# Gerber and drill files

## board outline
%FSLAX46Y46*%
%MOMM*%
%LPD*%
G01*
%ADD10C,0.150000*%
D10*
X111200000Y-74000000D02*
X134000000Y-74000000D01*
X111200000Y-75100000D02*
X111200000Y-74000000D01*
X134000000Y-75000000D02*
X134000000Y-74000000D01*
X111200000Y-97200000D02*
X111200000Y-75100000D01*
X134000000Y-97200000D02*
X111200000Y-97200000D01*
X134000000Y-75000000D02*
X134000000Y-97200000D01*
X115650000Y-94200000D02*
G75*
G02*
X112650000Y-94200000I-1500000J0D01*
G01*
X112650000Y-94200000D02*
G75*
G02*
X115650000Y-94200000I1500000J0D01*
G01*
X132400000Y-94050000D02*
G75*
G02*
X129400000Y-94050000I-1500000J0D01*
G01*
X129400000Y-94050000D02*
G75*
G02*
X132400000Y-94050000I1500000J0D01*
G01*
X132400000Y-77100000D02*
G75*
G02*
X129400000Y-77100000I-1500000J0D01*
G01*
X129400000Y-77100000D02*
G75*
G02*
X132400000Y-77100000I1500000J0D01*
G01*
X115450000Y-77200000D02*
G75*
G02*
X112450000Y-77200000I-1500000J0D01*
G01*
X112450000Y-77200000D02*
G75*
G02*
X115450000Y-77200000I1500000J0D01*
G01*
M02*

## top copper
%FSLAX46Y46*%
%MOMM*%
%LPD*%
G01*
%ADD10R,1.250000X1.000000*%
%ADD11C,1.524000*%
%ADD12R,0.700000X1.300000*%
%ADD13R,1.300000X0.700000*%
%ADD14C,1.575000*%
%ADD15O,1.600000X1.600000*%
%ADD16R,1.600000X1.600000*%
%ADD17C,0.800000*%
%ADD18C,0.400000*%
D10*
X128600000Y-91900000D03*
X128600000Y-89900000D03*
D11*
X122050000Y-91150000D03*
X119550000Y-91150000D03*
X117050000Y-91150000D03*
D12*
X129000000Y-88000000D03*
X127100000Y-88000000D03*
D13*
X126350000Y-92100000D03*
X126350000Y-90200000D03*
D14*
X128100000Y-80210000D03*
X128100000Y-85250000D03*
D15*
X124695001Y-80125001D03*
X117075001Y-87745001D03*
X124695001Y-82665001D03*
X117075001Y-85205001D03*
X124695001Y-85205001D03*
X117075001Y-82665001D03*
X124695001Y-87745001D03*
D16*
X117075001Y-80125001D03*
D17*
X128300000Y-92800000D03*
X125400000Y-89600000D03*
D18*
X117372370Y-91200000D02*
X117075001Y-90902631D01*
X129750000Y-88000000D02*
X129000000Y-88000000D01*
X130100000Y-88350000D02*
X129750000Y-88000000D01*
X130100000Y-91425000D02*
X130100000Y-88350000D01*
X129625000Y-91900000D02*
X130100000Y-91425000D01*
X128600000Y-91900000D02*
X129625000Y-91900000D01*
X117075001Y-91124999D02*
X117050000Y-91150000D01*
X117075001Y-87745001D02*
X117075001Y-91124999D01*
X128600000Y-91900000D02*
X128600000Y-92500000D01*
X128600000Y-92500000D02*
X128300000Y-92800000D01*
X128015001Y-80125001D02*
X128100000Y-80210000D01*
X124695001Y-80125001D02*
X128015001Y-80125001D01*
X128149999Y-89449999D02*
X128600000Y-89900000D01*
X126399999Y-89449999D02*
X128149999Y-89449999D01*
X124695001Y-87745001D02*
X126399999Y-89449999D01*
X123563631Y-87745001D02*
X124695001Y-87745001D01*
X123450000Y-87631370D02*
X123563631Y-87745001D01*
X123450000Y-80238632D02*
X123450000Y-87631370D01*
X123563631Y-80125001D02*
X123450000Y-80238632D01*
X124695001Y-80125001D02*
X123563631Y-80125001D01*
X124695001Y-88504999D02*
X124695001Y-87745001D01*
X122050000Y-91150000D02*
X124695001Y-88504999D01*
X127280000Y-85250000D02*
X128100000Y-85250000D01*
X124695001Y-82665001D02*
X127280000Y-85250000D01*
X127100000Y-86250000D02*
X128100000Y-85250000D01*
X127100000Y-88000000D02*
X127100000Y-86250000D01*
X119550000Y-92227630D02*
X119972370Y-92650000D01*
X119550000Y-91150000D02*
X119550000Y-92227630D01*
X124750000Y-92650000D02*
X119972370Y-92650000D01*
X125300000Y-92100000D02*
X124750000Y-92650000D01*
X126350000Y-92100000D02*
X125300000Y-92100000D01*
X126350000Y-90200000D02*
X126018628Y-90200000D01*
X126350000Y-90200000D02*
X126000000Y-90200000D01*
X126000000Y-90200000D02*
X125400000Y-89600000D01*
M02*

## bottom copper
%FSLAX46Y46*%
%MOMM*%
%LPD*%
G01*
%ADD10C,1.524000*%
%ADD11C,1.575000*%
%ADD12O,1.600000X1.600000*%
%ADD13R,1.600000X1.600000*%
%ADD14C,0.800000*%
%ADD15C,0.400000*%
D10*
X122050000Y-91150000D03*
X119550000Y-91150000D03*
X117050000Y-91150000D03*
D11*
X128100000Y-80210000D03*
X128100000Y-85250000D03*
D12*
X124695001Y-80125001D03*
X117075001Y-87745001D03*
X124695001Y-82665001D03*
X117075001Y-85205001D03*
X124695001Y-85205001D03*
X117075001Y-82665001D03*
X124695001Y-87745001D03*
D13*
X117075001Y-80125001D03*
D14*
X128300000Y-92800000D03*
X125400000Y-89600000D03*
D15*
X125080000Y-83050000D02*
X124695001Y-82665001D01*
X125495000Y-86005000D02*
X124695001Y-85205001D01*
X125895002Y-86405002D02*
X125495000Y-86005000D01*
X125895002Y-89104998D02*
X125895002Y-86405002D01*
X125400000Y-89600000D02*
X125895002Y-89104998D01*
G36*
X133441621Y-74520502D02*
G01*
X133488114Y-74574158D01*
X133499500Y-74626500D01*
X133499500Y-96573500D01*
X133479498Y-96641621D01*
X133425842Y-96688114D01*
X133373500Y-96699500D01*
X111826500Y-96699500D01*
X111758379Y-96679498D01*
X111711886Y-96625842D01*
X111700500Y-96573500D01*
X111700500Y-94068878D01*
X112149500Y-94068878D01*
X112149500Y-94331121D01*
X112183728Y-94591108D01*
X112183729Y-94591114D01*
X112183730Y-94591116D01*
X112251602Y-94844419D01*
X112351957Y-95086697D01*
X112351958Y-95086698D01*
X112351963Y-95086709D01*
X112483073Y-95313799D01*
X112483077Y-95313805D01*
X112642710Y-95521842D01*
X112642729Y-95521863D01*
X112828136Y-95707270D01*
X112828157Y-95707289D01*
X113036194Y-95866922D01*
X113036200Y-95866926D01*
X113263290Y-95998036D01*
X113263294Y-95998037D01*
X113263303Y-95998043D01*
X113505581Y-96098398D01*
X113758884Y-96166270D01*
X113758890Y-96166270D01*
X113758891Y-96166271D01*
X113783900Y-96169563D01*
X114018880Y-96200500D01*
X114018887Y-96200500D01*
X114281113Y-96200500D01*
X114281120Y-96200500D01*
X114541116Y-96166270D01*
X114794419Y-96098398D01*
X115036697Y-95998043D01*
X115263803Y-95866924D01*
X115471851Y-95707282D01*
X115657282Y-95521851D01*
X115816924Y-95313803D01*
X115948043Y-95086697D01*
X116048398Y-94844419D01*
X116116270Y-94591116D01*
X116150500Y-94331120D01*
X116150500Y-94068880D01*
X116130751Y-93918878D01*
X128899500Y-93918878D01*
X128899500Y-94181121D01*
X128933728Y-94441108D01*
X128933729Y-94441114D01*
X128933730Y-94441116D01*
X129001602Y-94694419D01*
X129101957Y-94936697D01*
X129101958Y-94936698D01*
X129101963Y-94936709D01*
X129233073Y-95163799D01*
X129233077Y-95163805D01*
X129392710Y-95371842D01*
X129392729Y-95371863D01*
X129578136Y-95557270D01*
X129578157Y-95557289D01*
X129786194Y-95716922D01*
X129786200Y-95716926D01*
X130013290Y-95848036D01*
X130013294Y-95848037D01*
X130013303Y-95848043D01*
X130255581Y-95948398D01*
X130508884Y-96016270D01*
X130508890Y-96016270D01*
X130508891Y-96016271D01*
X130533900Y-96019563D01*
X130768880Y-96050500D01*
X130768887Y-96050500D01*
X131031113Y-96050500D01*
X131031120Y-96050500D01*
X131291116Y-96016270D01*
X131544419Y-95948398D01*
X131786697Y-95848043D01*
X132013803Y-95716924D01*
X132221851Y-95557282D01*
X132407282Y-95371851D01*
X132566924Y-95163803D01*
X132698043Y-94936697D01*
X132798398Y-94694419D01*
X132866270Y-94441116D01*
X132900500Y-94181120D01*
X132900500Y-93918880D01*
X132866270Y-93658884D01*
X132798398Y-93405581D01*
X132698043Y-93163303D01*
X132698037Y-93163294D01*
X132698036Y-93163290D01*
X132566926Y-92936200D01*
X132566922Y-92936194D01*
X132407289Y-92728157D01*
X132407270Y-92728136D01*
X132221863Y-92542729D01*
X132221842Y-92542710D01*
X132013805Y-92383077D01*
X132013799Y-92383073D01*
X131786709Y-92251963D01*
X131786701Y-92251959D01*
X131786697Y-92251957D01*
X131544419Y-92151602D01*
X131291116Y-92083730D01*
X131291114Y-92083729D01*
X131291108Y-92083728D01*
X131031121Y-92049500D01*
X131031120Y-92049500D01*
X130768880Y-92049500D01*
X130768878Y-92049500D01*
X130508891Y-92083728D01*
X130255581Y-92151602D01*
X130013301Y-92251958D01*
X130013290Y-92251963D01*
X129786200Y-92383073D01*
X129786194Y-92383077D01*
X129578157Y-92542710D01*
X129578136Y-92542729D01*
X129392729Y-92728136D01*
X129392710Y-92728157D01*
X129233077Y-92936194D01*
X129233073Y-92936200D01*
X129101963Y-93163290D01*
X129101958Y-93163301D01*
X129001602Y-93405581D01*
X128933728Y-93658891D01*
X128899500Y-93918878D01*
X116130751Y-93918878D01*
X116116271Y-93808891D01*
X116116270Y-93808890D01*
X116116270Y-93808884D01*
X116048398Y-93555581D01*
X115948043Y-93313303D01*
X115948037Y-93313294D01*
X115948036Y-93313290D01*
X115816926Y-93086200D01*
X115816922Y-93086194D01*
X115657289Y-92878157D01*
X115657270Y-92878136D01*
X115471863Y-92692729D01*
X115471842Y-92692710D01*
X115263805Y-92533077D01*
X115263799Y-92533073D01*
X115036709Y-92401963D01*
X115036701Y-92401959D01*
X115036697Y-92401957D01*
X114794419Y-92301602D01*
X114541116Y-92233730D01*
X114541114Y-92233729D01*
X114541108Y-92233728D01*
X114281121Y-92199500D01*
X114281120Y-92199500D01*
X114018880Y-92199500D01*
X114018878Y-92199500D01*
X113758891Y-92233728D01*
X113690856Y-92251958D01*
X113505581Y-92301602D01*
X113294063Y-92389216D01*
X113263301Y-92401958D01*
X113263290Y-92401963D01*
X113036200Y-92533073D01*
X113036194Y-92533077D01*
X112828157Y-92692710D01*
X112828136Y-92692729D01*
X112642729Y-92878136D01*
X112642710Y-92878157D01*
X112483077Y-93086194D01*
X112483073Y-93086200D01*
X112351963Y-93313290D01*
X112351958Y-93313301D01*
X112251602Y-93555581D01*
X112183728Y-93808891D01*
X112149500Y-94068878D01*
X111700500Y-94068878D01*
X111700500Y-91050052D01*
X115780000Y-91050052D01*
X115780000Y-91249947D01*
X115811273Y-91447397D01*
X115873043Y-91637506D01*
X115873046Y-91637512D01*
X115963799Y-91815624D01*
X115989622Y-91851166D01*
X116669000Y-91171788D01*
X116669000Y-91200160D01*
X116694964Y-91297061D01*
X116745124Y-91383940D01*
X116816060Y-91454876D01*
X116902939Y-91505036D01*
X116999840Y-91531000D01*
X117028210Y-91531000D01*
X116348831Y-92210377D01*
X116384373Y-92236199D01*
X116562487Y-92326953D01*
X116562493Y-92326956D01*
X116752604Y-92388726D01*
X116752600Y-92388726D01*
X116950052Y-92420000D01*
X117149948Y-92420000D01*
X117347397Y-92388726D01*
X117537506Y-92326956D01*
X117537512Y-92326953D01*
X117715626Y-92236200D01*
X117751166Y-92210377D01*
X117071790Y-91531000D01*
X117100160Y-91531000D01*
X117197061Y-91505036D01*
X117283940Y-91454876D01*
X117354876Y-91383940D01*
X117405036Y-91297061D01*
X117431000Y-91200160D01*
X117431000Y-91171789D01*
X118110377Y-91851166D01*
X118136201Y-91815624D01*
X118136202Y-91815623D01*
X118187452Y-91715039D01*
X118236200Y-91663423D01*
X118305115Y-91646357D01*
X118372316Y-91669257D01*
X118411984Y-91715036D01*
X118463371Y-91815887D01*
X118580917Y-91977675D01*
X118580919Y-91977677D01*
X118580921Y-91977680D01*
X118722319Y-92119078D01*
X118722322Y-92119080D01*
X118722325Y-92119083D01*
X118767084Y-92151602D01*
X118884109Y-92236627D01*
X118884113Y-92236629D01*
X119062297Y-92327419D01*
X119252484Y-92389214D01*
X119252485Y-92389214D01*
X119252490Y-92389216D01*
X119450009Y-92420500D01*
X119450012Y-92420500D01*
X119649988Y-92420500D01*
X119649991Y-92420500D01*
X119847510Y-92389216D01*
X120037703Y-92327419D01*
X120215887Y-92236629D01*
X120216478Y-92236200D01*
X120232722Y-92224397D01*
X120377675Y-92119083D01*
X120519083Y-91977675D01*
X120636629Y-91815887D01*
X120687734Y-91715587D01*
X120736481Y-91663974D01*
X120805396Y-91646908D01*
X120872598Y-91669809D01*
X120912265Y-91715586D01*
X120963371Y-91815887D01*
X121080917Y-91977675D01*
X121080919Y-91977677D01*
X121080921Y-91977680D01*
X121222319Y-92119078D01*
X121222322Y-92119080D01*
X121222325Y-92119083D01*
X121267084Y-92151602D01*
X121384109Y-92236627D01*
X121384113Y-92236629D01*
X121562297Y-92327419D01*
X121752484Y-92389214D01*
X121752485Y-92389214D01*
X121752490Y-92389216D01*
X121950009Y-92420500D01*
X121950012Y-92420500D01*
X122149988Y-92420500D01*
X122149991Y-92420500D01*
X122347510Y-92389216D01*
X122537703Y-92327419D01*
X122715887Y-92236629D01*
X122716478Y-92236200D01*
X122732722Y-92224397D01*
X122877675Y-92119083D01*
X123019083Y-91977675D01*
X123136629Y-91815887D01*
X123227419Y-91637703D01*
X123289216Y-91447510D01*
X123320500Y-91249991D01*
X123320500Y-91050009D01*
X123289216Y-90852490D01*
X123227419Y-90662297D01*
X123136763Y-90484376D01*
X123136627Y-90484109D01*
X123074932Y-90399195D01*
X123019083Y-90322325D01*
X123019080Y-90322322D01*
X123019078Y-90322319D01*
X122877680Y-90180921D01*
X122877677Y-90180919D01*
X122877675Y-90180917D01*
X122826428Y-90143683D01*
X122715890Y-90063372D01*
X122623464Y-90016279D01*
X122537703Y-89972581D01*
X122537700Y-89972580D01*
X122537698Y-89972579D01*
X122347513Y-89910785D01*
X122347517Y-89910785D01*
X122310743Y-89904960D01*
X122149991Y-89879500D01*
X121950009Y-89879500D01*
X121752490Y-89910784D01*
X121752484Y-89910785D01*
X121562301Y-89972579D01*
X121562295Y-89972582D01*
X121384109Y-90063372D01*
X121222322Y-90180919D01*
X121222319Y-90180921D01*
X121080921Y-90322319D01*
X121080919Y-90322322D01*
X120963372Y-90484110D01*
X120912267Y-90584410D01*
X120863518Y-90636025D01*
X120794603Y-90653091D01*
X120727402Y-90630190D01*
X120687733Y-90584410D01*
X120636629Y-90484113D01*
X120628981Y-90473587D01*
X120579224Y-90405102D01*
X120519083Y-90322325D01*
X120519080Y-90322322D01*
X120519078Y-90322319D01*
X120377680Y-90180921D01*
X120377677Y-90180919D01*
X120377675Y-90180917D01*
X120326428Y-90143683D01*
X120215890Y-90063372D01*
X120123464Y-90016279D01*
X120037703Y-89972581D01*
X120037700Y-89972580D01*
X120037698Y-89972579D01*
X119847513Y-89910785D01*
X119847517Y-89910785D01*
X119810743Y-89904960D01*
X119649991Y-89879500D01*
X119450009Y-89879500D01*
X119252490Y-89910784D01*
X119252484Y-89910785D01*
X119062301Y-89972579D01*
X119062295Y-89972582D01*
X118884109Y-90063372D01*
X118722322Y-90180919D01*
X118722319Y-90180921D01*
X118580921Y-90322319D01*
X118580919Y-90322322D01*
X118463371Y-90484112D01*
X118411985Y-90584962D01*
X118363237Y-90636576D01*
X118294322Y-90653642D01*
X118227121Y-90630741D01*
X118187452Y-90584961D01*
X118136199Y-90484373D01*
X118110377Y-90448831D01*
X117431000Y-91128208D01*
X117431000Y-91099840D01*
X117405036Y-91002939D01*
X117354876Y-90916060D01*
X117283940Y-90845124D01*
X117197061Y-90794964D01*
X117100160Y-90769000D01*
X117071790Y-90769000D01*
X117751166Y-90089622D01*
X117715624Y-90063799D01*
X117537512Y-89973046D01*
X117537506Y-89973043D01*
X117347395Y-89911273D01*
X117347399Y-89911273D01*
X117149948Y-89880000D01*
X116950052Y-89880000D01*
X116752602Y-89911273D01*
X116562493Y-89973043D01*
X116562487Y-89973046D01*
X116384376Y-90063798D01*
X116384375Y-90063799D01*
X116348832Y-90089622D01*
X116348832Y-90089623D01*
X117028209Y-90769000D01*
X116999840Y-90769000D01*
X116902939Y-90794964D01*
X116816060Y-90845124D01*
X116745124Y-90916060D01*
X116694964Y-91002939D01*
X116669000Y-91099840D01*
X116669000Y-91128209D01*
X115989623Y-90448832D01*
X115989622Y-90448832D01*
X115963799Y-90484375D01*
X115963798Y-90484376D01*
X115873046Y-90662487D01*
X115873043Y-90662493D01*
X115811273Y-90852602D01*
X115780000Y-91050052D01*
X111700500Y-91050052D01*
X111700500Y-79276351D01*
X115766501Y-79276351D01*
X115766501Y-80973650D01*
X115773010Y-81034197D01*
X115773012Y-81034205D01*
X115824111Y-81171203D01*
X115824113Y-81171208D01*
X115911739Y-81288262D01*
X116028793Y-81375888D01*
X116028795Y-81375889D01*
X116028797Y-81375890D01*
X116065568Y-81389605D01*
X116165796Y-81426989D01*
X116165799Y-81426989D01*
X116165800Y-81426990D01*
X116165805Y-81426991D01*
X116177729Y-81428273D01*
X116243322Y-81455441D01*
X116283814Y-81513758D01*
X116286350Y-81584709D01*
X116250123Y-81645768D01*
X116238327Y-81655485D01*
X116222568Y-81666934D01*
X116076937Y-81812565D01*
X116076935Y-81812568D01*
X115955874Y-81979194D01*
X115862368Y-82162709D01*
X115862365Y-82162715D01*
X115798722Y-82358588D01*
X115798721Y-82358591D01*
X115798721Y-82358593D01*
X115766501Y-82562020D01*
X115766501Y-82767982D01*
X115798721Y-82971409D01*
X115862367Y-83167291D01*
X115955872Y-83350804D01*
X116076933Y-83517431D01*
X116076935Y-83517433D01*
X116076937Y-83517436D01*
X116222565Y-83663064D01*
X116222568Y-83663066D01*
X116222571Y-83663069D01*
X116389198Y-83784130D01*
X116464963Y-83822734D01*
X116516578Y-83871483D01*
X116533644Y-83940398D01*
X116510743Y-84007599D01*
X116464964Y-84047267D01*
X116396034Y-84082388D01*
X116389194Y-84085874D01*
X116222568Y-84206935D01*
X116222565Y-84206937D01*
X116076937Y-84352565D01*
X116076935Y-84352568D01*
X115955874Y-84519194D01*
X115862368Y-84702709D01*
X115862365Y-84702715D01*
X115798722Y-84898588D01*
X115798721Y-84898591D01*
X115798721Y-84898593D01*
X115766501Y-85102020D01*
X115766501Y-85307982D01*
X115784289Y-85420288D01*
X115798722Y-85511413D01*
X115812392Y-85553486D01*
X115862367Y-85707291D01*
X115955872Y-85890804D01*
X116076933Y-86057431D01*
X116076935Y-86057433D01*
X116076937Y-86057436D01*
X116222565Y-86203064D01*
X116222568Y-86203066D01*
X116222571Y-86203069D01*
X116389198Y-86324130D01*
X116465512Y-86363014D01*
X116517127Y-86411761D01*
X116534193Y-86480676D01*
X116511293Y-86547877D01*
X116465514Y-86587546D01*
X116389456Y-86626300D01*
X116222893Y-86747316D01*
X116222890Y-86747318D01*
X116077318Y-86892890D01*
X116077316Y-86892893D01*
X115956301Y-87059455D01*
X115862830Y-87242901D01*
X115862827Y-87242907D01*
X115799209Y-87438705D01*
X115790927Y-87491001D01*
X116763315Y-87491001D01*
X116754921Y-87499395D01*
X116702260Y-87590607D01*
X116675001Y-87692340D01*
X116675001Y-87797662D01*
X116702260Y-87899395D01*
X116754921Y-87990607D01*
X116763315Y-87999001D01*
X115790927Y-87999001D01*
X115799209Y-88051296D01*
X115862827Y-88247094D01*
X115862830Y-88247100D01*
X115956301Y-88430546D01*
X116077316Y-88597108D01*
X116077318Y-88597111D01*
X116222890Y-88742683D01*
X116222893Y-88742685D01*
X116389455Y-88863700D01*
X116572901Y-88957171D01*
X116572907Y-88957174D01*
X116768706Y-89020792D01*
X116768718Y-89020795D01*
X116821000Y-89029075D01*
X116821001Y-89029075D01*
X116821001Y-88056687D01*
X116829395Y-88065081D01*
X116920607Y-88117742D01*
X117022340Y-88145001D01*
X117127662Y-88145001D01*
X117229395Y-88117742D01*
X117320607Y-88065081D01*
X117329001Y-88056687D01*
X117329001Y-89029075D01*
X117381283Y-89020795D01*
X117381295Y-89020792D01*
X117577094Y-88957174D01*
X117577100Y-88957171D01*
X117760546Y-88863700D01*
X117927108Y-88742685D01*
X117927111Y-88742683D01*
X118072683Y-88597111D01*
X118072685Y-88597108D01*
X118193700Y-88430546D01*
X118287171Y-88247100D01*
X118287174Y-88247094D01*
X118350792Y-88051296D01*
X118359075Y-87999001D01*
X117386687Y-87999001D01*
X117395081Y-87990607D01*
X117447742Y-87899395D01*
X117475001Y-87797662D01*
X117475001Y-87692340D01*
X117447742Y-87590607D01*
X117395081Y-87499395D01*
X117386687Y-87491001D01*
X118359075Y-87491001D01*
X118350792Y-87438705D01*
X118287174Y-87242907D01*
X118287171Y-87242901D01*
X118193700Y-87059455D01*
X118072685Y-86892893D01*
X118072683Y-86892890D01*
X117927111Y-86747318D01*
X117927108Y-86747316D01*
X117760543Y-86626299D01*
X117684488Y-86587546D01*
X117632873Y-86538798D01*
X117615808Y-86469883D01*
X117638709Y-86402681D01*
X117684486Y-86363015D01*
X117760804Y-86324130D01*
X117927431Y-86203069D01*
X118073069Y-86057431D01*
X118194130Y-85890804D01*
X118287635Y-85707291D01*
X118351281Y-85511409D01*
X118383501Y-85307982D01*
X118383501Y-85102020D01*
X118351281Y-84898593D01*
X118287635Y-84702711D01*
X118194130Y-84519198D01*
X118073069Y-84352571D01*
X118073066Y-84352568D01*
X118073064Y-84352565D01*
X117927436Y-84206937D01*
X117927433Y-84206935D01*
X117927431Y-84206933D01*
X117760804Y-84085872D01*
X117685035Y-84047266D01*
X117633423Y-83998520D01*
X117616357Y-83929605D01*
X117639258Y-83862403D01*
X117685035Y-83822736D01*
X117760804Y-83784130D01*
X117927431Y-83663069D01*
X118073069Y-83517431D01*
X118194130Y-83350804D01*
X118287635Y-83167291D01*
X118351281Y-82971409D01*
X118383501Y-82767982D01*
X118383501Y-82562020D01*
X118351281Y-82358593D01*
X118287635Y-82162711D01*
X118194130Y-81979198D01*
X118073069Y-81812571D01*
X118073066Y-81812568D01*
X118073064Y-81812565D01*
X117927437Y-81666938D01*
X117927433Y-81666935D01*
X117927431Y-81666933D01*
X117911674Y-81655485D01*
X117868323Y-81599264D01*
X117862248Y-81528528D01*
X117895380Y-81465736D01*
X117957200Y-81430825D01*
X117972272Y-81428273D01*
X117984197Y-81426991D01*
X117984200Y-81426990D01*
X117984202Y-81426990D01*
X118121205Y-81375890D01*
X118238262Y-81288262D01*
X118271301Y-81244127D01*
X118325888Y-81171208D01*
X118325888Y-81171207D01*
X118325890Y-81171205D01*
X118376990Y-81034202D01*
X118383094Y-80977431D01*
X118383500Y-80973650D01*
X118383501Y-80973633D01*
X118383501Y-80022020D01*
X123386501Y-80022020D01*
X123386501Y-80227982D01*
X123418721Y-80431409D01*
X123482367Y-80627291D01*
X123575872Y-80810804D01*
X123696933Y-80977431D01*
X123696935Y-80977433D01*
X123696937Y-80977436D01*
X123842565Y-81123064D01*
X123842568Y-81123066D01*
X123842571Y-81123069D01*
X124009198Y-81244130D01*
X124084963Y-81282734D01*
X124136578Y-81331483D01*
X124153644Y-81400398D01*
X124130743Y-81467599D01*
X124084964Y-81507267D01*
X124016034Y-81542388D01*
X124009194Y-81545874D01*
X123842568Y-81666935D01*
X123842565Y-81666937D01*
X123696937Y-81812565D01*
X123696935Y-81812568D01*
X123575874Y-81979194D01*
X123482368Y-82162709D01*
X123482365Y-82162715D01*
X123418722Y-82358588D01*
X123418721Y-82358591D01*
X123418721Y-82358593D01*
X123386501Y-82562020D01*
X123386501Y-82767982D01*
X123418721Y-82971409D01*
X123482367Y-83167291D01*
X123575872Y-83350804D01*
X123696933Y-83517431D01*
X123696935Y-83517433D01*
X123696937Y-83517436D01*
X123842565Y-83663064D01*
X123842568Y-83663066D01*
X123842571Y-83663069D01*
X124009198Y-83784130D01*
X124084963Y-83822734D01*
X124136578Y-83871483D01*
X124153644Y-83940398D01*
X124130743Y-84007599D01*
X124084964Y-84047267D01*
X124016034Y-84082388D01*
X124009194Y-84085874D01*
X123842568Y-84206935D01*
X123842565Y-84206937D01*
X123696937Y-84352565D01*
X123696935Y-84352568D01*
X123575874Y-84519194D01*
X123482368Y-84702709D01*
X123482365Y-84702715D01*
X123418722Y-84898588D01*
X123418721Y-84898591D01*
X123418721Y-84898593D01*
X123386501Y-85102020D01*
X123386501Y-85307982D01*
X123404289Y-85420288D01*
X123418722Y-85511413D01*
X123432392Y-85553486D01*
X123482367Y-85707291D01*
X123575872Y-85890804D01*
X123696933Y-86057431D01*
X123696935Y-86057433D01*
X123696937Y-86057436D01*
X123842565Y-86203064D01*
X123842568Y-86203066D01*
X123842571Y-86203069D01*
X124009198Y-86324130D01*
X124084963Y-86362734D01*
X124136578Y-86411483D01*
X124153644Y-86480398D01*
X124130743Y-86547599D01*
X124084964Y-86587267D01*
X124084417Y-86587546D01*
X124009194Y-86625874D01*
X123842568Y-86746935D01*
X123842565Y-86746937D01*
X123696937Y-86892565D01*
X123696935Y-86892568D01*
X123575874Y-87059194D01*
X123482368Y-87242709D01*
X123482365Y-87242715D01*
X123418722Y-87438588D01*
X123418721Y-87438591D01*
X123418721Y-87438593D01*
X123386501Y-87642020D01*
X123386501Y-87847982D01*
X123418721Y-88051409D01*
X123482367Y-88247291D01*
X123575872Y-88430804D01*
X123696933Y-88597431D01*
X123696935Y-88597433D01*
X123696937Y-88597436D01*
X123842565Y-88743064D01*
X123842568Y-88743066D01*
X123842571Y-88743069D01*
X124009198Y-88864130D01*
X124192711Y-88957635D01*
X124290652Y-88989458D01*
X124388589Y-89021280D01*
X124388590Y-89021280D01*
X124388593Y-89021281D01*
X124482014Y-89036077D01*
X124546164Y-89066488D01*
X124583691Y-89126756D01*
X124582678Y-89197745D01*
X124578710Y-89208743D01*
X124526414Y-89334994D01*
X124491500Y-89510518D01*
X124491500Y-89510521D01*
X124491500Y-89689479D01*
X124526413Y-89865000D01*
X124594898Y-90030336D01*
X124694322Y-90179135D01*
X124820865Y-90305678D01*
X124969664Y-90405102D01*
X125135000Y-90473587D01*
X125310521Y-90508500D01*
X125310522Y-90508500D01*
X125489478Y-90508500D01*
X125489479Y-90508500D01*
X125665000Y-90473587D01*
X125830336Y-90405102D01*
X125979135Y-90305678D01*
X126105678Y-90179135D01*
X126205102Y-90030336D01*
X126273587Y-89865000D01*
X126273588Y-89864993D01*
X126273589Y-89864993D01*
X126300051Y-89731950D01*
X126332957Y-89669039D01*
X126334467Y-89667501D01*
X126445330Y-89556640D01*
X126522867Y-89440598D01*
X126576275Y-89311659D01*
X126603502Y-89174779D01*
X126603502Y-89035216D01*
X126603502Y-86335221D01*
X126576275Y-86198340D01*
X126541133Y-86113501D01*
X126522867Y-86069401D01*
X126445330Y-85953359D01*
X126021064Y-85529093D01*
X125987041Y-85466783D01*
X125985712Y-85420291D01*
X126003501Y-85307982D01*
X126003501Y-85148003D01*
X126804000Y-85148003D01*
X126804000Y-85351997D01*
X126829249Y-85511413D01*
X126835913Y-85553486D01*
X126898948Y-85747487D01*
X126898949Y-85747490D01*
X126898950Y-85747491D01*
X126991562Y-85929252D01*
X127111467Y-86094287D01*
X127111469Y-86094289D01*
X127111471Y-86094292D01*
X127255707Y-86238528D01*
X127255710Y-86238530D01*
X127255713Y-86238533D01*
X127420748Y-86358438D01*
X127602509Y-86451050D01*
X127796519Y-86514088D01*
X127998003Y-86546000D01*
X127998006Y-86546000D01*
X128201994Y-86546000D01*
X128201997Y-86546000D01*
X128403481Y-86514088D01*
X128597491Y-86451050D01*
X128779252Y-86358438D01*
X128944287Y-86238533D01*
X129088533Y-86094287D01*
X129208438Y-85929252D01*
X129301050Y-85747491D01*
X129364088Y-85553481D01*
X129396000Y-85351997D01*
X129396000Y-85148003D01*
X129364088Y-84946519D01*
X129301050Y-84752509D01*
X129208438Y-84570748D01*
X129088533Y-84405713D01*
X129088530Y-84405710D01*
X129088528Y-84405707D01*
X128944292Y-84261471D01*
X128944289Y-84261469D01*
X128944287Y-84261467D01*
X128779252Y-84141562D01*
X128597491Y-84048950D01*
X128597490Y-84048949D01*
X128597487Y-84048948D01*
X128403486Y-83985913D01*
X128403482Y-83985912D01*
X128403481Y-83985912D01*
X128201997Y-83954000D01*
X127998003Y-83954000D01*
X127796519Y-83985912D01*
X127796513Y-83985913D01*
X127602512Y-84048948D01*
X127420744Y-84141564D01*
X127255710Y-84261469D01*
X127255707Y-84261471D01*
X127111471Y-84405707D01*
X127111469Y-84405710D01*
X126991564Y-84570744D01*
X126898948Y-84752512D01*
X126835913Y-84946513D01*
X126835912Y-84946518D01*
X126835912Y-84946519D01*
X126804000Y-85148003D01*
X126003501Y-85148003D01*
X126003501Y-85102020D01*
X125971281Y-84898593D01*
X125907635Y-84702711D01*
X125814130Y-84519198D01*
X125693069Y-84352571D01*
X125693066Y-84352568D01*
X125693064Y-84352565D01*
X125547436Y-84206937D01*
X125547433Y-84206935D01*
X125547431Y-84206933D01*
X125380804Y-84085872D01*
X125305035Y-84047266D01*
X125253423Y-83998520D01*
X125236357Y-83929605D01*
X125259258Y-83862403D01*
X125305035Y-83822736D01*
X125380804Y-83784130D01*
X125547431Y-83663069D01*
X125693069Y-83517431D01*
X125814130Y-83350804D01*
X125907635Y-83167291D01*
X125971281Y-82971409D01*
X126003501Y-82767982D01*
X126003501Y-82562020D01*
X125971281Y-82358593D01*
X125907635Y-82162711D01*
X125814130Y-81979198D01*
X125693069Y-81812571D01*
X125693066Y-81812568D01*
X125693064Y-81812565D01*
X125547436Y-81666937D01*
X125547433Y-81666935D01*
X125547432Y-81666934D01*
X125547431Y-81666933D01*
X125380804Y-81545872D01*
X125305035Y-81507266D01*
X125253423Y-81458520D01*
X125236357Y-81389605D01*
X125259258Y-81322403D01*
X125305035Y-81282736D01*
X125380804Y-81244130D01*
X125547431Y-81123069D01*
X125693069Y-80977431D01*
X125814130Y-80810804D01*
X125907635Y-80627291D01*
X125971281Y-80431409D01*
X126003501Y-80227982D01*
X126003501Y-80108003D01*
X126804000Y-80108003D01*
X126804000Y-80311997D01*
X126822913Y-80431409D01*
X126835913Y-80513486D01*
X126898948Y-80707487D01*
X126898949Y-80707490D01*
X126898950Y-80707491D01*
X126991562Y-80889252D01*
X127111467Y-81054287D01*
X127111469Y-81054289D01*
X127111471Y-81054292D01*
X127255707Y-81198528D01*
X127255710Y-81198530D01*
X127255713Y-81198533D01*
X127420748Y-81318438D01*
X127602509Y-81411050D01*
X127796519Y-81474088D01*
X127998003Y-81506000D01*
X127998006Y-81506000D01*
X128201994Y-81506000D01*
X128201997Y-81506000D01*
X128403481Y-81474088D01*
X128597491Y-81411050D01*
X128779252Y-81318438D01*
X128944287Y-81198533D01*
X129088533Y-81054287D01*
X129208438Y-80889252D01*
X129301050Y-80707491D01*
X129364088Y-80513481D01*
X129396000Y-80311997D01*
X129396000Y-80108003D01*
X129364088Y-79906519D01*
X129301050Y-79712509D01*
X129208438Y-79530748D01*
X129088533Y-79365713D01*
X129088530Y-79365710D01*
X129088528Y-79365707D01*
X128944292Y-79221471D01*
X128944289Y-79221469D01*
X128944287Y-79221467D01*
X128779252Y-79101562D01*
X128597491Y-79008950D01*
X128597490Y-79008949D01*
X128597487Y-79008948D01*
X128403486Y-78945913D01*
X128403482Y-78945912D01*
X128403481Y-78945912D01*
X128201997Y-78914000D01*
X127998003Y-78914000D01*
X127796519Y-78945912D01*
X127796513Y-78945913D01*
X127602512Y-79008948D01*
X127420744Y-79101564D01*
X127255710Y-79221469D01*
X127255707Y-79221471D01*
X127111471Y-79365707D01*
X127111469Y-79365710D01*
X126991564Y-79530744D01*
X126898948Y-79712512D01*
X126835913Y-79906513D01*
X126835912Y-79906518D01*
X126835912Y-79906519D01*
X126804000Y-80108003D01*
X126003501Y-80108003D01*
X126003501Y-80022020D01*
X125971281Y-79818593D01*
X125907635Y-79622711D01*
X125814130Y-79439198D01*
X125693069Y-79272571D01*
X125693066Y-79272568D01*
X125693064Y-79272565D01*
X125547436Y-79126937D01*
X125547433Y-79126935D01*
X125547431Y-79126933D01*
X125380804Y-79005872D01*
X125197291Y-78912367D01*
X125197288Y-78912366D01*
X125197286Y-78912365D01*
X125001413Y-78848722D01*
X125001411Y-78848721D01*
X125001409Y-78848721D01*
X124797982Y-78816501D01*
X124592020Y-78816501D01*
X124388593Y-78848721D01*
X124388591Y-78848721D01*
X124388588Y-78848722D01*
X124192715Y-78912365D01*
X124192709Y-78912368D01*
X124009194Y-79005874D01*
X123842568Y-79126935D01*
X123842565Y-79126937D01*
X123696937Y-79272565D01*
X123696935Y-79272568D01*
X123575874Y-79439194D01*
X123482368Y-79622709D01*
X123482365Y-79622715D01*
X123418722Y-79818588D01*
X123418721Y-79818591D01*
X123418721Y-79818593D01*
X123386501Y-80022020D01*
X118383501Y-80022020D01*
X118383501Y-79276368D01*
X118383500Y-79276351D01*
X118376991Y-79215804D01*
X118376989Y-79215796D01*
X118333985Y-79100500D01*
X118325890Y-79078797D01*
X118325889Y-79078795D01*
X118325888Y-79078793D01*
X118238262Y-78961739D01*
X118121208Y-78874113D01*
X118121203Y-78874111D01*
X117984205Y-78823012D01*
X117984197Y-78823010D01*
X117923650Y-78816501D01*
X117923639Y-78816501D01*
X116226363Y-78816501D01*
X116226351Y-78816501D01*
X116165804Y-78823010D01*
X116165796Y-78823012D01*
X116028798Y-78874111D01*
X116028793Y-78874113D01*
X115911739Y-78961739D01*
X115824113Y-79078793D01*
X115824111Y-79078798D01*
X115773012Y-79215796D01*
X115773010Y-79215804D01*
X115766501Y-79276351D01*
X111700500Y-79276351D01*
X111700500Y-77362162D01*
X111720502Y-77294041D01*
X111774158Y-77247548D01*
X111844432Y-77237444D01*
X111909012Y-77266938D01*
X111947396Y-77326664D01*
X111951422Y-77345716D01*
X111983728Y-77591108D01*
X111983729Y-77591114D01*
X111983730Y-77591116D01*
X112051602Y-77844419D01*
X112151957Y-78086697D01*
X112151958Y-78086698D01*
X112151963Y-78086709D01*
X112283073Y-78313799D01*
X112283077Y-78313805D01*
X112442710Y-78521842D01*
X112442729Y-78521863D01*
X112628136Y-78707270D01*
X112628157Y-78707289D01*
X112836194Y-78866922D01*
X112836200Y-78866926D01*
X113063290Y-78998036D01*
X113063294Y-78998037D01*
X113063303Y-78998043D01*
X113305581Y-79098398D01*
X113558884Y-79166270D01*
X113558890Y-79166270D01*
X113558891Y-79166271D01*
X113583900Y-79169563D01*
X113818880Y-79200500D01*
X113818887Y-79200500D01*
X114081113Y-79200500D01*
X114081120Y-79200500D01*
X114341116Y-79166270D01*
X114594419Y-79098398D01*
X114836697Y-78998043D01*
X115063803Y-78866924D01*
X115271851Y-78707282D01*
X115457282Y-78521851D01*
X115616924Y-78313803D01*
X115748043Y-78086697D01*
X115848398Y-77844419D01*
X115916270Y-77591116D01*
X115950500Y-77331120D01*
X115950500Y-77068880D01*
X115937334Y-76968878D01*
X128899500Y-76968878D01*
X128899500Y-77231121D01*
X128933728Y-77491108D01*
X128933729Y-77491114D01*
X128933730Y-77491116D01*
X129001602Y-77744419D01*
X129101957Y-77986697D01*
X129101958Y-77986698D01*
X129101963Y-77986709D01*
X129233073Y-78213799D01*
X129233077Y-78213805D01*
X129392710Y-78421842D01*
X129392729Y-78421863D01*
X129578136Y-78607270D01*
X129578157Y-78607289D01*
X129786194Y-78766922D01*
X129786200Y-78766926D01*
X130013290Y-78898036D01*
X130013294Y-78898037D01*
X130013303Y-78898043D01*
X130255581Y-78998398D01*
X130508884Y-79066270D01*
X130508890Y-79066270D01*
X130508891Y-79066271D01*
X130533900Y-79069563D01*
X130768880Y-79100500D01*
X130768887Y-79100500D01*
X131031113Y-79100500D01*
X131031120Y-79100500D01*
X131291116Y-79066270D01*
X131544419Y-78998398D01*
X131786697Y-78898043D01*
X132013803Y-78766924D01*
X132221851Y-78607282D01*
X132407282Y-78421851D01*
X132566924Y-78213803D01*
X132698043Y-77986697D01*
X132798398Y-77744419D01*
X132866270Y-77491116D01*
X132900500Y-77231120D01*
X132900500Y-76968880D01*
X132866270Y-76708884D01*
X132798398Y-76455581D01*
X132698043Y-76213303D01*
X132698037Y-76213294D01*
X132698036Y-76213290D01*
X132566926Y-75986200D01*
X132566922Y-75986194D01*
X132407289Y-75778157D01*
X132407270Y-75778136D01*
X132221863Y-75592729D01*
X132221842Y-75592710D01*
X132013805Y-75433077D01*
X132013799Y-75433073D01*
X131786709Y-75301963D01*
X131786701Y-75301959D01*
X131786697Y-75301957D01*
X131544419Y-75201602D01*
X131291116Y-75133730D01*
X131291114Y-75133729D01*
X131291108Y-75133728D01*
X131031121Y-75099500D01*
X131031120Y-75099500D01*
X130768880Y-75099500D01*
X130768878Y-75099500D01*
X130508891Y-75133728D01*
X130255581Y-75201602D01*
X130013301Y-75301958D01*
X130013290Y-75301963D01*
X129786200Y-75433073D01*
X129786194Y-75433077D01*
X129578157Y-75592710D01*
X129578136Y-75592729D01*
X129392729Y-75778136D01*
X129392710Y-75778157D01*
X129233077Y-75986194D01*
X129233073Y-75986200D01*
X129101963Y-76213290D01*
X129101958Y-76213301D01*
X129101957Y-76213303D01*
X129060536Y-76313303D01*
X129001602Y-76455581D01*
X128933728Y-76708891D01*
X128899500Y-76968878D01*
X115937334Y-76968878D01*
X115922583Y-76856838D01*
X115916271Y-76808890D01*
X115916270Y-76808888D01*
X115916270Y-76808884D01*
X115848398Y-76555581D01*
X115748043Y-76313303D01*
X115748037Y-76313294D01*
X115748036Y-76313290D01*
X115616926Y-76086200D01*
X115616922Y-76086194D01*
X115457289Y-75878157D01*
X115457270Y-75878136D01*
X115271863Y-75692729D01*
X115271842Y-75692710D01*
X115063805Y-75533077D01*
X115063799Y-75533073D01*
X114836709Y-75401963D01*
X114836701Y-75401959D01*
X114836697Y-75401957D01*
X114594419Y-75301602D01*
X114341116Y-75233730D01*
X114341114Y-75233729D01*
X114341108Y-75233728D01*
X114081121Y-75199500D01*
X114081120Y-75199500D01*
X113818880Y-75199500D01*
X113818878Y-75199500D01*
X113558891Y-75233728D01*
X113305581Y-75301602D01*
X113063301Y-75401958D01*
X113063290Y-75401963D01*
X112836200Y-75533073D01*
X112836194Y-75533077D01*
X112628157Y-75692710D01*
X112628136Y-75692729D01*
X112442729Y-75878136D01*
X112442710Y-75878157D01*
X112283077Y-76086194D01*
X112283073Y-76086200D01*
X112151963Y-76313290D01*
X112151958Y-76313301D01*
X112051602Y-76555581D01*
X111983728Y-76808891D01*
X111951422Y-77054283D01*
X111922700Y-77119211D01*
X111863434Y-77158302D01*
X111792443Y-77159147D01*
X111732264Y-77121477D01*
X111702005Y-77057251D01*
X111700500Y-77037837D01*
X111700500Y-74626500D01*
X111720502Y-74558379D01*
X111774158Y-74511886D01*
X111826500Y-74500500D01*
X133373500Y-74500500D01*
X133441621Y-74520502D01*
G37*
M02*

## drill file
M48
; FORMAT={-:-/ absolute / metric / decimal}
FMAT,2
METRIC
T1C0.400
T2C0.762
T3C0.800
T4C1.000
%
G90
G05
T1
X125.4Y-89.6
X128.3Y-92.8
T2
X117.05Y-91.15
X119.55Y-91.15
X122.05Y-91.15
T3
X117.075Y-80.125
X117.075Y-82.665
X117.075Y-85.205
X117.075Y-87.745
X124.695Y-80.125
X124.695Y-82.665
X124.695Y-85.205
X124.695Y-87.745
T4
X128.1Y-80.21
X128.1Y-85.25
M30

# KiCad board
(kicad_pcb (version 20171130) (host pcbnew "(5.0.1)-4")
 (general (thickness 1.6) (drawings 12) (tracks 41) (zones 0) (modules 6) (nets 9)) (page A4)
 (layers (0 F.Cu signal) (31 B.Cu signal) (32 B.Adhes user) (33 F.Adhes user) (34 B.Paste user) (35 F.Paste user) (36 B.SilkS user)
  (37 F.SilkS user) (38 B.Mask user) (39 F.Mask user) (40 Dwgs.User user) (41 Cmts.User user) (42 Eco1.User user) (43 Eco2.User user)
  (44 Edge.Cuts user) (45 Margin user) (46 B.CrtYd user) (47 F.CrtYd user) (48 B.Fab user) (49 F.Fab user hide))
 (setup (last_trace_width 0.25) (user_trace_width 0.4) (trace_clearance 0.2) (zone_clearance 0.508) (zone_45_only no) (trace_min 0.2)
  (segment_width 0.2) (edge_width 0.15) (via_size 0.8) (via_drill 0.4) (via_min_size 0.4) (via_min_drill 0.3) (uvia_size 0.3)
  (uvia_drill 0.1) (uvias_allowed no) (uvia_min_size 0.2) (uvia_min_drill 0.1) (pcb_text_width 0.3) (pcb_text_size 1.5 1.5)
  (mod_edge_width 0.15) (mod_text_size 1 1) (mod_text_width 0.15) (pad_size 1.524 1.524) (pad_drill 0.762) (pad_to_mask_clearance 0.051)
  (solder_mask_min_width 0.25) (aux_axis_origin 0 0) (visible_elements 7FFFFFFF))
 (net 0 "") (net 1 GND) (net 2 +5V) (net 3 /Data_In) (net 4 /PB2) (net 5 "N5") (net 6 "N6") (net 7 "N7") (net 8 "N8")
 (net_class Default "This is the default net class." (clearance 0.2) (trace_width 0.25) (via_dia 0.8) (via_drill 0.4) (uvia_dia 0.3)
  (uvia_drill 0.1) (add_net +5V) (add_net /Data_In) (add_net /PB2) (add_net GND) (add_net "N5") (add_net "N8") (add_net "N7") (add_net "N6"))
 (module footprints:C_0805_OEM (layer F.Cu) (at 128.6 90.9 90)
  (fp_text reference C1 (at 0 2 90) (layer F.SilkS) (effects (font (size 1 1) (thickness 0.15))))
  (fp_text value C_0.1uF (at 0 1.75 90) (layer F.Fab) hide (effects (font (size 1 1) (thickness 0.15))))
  (pad 1 smd rect (at -1 0 90) (size 1 1.25) (layers F.Cu F.Paste F.Mask) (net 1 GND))
  (pad 2 smd rect (at 1 0 90) (size 1 1.25) (layers F.Cu F.Paste F.Mask) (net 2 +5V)))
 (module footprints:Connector (layer F.Cu) (at 119.55 91.15 180)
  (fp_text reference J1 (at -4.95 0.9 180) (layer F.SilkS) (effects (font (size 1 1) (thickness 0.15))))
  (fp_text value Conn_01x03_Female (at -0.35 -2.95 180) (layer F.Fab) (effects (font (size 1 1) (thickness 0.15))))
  (pad 1 thru_hole circle (at -2.5 0 180) (size 1.524 1.524) (drill 0.762) (layers *.Cu *.Mask) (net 2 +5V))
  (pad 2 thru_hole circle (at 0 0 180) (size 1.524 1.524) (drill 0.762) (layers *.Cu *.Mask) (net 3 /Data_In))
  (pad 3 thru_hole circle (at 2.5 0 180) (size 1.524 1.524) (drill 0.762) (layers *.Cu *.Mask) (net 1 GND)))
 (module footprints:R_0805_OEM (layer F.Cu) (at 128.05 88)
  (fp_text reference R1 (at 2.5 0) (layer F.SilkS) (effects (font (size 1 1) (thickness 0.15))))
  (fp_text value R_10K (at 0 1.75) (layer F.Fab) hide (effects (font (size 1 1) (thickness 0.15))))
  (pad 2 smd rect (at 0.95 0) (size 0.7 1.3) (layers F.Cu F.Paste F.Mask) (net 1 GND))
  (pad 1 smd rect (at -0.95 0) (size 0.7 1.3) (layers F.Cu F.Paste F.Mask) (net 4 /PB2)))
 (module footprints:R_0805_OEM (layer F.Cu) (at 126.35 91.15 90)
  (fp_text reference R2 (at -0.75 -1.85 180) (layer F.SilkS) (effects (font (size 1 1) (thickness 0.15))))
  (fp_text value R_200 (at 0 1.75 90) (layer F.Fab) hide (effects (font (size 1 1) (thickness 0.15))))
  (pad 1 smd rect (at -0.95 0 90) (size 0.7 1.3) (layers F.Cu F.Paste F.Mask) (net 3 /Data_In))
  (pad 2 smd rect (at 0.95 0 90) (size 0.7 1.3) (layers F.Cu F.Paste F.Mask) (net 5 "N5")))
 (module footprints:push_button (layer F.Cu) (at 128.1 82.75 270)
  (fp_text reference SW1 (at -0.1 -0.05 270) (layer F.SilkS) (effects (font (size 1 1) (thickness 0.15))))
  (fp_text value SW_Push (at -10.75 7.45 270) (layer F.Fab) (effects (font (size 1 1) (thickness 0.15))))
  (pad 1 thru_hole circle (at -2.54 0 270) (size 1.575 1.575) (drill 1) (layers *.Cu *.Mask) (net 2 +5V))
  (pad 2 thru_hole circle (at 2.5 0 270) (size 1.575 1.575) (drill 1) (layers *.Cu *.Mask) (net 4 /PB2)))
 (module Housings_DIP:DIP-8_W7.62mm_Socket (layer F.Cu) (at 117.075001 80.125001)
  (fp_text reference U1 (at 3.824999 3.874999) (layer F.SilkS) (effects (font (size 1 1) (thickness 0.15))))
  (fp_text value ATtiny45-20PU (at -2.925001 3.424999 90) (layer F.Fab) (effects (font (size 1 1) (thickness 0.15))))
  (pad 8 thru_hole oval (at 7.62 0) (size 1.6 1.6) (drill 0.8) (layers *.Cu *.Mask) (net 2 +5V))
  (pad 4 thru_hole oval (at 0 7.62) (size 1.6 1.6) (drill 0.8) (layers *.Cu *.Mask) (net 1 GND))
  (pad 7 thru_hole oval (at 7.62 2.54) (size 1.6 1.6) (drill 0.8) (layers *.Cu *.Mask) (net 4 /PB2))
  (pad 3 thru_hole oval (at 0 5.08) (size 1.6 1.6) (drill 0.8) (layers *.Cu *.Mask) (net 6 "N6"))
  (pad 6 thru_hole oval (at 7.62 5.08) (size 1.6 1.6) (drill 0.8) (layers *.Cu *.Mask) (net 5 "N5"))
  (pad 2 thru_hole oval (at 0 2.54) (size 1.6 1.6) (drill 0.8) (layers *.Cu *.Mask) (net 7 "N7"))
  (pad 5 thru_hole oval (at 7.62 7.62) (size 1.6 1.6) (drill 0.8) (layers *.Cu *.Mask) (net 2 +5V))
  (pad 1 thru_hole rect (at 0 0) (size 1.6 1.6) (drill 0.8) (layers *.Cu *.Mask) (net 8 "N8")))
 (gr_line (start 111.2 74) (end 134 74) (layer Edge.Cuts) (width 0.15))
 (gr_line (start 111.2 75.1) (end 111.2 74) (layer Edge.Cuts) (width 0.15))
 (gr_line (start 134 75) (end 134 74) (layer Edge.Cuts) (width 0.15))
 (gr_line (start 111.2 97.2) (end 111.2 75.1) (layer Edge.Cuts) (width 0.15))
 (gr_line (start 134 97.2) (end 111.2 97.2) (layer Edge.Cuts) (width 0.15))
 (gr_line (start 134 75) (end 134 97.2) (layer Edge.Cuts) (width 0.15))
 (gr_circle (center 114.15 94.2) (end 115.65 94.2) (layer Edge.Cuts) (width 0.15))
 (gr_circle (center 130.9 94.05) (end 132.4 94.05) (layer Edge.Cuts) (width 0.15))
 (gr_circle (center 130.9 77.1) (end 132.4 77.1) (layer Edge.Cuts) (width 0.15))
 (gr_circle (center 113.95 77.2) (end 115.45 77.2) (layer Edge.Cuts) (width 0.15))
 (segment (start 117.37237 91.2) (end 117.075001 90.902631) (width 0.4) (layer F.Cu) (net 1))
 (segment (start 129.75 88) (end 129 88) (width 0.4) (layer F.Cu) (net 1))
 (segment (start 130.1 88.35) (end 129.75 88) (width 0.4) (layer F.Cu) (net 1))
 (segment (start 130.1 91.425) (end 130.1 88.35) (width 0.4) (layer F.Cu) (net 1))
 (segment (start 129.625 91.9) (end 130.1 91.425) (width 0.4) (layer F.Cu) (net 1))
 (segment (start 128.6 91.9) (end 129.625 91.9) (width 0.4) (layer F.Cu) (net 1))
 (segment (start 117.075001 91.124999) (end 117.05 91.15) (width 0.4) (layer F.Cu) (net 1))
 (segment (start 117.075001 87.745001) (end 117.075001 91.124999) (width 0.4) (layer F.Cu) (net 1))
 (via (at 128.3 92.8) (size 0.8) (drill 0.4) (layers F.Cu B.Cu) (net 1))
 (segment (start 128.6 91.9) (end 128.6 92.5) (width 0.4) (layer F.Cu) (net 1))
 (segment (start 128.6 92.5) (end 128.3 92.8) (width 0.4) (layer F.Cu) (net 1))
 (segment (start 128.015001 80.125001) (end 128.1 80.21) (width 0.4) (layer F.Cu) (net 2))
 (segment (start 124.695001 80.125001) (end 128.015001 80.125001) (width 0.4) (layer F.Cu) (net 2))
 (segment (start 128.149999 89.449999) (end 128.6 89.9) (width 0.4) (layer F.Cu) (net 2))
 (segment (start 126.399999 89.449999) (end 128.149999 89.449999) (width 0.4) (layer F.Cu) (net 2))
 (segment (start 124.695001 87.745001) (end 126.399999 89.449999) (width 0.4) (layer F.Cu) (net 2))
 (segment (start 123.563631 87.745001) (end 124.695001 87.745001) (width 0.4) (layer F.Cu) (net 2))
 (segment (start 123.45 87.63137) (end 123.563631 87.745001) (width 0.4) (layer F.Cu) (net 2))
 (segment (start 123.45 80.238632) (end 123.45 87.63137) (width 0.4) (layer F.Cu) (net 2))
 (segment (start 123.563631 80.125001) (end 123.45 80.238632) (width 0.4) (layer F.Cu) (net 2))
 (segment (start 124.695001 80.125001) (end 123.563631 80.125001) (width 0.4) (layer F.Cu) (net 2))
 (segment (start 124.695001 88.504999) (end 124.695001 87.745001) (width 0.4) (layer F.Cu) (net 2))
 (segment (start 122.05 91.15) (end 124.695001 88.504999) (width 0.4) (layer F.Cu) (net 2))
 (segment (start 125.08 83.05) (end 124.695001 82.665001) (width 0.4) (layer B.Cu) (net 4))
 (segment (start 127.28 85.25) (end 128.1 85.25) (width 0.4) (layer F.Cu) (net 4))
 (segment (start 124.695001 82.665001) (end 127.28 85.25) (width 0.4) (layer F.Cu) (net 4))
 (segment (start 127.1 86.25) (end 128.1 85.25) (width 0.4) (layer F.Cu) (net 4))
 (segment (start 127.1 88) (end 127.1 86.25) (width 0.4) (layer F.Cu) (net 4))
 (segment (start 119.55 92.22763) (end 119.97237 92.65) (width 0.4) (layer F.Cu) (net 3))
 (segment (start 119.55 91.15) (end 119.55 92.22763) (width 0.4) (layer F.Cu) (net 3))
 (segment (start 124.75 92.65) (end 119.97237 92.65) (width 0.4) (layer F.Cu) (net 3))
 (segment (start 125.3 92.1) (end 124.75 92.65) (width 0.4) (layer F.Cu) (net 3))
 (segment (start 126.35 92.1) (end 125.3 92.1) (width 0.4) (layer F.Cu) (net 3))
 (segment (start 126.35 90.2) (end 126.018628 90.2) (width 0.4) (layer F.Cu) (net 5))
 (via (at 125.4 89.6) (size 0.8) (drill 0.4) (layers F.Cu B.Cu) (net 5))
 (segment (start 126.35 90.2) (end 126 90.2) (width 0.4) (layer F.Cu) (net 5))
 (segment (start 126 90.2) (end 125.4 89.6) (width 0.4) (layer F.Cu) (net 5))
 (segment (start 125.495 86.005) (end 124.695001 85.205001) (width 0.4) (layer B.Cu) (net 5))
 (segment (start 125.895002 86.405002) (end 125.495 86.005) (width 0.4) (layer B.Cu) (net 5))
 (segment (start 125.895002 89.104998) (end 125.895002 86.405002) (width 0.4) (layer B.Cu) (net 5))
 (segment (start 125.4 89.6) (end 125.895002 89.104998) (width 0.4) (layer B.Cu) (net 5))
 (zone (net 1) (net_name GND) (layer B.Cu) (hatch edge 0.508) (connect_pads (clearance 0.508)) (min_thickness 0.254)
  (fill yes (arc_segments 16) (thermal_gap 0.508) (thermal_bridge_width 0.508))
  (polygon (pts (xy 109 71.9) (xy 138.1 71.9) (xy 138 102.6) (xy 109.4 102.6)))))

